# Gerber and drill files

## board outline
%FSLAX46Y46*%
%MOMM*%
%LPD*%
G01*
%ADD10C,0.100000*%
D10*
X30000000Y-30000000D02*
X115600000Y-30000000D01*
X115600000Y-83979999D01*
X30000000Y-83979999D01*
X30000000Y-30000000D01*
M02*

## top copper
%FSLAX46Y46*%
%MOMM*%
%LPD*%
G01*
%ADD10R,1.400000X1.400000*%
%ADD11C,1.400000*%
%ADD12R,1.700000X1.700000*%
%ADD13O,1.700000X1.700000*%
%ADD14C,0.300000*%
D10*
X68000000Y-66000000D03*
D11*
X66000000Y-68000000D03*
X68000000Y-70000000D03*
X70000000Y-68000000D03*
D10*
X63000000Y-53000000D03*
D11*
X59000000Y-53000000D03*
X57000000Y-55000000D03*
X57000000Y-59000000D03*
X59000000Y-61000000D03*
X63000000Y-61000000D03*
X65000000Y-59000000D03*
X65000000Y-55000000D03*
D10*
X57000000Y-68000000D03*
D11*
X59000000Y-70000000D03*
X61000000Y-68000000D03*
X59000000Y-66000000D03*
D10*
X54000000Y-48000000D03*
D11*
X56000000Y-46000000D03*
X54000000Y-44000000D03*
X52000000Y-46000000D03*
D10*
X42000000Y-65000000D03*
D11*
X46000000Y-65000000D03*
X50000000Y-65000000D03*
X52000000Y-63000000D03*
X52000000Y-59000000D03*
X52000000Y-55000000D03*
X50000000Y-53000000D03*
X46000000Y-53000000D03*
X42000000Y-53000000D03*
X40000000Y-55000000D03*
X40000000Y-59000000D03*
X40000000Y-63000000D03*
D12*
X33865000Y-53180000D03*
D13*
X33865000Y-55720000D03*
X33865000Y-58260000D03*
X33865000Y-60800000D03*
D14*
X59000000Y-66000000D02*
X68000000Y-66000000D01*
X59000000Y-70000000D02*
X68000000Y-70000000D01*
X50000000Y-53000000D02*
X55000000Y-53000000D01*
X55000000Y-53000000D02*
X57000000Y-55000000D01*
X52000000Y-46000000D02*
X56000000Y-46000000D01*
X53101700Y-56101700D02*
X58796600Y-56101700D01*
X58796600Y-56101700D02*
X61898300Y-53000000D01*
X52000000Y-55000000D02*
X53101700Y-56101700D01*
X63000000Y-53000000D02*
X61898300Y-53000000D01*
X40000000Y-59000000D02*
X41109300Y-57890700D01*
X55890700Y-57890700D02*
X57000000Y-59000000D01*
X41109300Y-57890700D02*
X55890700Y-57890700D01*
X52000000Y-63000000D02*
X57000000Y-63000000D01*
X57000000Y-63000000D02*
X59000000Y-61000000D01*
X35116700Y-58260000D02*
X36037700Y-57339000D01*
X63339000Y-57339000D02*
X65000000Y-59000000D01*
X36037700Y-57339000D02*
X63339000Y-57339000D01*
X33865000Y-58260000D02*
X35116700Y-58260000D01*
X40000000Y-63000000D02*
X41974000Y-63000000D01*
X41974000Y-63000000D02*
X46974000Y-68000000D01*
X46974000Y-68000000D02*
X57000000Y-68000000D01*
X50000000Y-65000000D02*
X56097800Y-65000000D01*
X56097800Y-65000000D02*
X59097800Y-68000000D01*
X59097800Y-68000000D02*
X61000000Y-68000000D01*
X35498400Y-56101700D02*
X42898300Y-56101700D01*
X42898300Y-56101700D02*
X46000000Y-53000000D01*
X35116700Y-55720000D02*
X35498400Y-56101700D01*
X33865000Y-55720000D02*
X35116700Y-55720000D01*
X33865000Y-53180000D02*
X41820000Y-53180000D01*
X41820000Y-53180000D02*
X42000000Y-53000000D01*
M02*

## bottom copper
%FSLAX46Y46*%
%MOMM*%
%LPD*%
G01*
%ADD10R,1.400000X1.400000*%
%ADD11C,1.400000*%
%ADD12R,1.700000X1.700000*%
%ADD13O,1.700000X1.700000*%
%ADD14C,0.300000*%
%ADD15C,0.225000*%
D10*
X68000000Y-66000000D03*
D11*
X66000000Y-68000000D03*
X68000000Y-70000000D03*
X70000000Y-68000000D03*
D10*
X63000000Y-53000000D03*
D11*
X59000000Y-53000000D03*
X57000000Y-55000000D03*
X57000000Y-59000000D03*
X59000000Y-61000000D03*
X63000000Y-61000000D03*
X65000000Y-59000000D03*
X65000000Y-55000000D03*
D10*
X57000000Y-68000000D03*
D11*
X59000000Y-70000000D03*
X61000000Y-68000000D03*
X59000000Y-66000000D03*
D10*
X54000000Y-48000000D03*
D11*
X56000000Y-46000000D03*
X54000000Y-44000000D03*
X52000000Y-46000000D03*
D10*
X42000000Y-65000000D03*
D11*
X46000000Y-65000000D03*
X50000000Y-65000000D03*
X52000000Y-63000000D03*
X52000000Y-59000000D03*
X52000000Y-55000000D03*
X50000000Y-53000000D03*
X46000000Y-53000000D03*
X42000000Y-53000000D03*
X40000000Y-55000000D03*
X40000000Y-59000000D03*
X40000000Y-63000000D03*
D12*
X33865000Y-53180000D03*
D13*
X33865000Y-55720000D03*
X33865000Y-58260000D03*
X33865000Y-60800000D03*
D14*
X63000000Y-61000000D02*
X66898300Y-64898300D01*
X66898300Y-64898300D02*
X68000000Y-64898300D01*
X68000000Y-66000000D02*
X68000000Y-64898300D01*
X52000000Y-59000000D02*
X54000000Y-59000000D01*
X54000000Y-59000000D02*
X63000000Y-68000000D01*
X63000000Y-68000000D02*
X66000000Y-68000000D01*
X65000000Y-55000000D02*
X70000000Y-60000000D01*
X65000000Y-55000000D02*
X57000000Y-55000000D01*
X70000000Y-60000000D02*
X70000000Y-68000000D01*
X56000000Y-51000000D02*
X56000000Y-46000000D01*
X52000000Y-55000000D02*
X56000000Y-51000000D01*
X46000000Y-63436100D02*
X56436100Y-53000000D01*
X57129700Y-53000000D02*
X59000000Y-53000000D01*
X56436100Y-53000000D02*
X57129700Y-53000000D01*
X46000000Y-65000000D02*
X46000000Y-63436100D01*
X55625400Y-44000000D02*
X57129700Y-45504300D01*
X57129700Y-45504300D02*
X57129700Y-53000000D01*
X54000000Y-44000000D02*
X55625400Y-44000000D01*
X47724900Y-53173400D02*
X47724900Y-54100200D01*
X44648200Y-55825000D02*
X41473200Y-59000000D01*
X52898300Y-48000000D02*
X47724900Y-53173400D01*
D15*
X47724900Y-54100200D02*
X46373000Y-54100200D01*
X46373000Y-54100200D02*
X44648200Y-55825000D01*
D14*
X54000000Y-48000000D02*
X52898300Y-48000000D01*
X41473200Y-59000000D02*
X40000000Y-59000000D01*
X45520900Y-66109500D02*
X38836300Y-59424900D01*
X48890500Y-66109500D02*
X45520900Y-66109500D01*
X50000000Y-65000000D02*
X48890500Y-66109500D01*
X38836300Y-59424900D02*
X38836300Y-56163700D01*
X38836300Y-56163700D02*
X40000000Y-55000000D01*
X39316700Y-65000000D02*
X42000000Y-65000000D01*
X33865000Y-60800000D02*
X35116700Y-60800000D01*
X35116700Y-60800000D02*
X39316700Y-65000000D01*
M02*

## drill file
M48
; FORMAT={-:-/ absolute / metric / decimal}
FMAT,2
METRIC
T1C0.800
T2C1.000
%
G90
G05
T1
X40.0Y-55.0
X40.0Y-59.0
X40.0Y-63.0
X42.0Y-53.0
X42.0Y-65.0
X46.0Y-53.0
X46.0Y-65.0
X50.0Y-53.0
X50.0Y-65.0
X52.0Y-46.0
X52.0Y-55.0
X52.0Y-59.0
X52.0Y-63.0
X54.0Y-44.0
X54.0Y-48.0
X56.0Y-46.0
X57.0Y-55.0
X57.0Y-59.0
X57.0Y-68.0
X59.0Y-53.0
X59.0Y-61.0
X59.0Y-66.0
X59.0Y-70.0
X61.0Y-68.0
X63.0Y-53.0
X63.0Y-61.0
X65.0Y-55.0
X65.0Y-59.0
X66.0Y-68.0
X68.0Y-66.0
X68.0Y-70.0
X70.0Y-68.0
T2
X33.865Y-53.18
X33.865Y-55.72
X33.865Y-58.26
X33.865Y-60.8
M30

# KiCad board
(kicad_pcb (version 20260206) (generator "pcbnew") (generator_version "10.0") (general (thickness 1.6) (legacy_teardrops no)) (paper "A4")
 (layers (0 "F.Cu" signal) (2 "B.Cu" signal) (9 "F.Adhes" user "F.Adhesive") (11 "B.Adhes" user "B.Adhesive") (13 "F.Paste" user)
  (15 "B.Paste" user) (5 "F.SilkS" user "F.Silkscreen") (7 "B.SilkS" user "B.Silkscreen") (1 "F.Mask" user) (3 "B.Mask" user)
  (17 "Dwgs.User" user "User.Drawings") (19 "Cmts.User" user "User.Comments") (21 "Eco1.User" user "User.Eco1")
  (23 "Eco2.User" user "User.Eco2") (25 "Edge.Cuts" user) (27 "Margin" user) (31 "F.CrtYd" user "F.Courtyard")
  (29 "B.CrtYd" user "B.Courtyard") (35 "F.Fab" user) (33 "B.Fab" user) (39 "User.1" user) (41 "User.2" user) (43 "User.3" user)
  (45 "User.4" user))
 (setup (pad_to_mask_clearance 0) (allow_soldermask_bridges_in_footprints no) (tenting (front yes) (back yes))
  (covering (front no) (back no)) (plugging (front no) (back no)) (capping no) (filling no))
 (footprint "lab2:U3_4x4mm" (layer "F.Cu") (at 68 68 -90)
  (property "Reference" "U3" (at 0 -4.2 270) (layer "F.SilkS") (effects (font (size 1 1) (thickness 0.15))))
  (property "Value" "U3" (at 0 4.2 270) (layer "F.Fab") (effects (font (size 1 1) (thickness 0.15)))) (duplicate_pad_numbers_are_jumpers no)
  (pad "1" thru_hole rect (at -2 0 270) (size 1.4 1.4) (drill 0.8) (layers "*.Cu" "*.Mask") (remove_unused_layers no) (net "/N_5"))
  (pad "2" thru_hole circle (at 0 2 270) (size 1.4 1.4) (drill 0.8) (layers "*.Cu" "*.Mask") (remove_unused_layers no) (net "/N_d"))
  (pad "3" thru_hole circle (at 2 0 270) (size 1.4 1.4) (drill 0.8) (layers "*.Cu" "*.Mask") (remove_unused_layers no) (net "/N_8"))
  (pad "4" thru_hole circle (at 0 -2 270) (size 1.4 1.4) (drill 0.8) (layers "*.Cu" "*.Mask") (remove_unused_layers no) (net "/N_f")))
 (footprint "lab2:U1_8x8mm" (layer "F.Cu") (at 61 57 -90)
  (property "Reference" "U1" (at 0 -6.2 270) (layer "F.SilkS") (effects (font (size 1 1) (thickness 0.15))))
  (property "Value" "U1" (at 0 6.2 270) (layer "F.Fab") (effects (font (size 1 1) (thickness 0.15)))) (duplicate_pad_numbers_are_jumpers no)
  (pad "1" thru_hole rect (at -4 -2 270) (size 1.4 1.4) (drill 0.8) (layers "*.Cu" "*.Mask") (remove_unused_layers no) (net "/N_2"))
  (pad "2" thru_hole circle (at -4 2 270) (size 1.4 1.4) (drill 0.8) (layers "*.Cu" "*.Mask") (remove_unused_layers no) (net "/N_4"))
  (pad "3" thru_hole circle (at -2 4 270) (size 1.4 1.4) (drill 0.8) (layers "*.Cu" "*.Mask") (remove_unused_layers no) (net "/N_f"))
  (pad "4" thru_hole circle (at 2 4 270) (size 1.4 1.4) (drill 0.8) (layers "*.Cu" "*.Mask") (remove_unused_layers no) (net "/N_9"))
  (pad "5" thru_hole circle (at 4 2 270) (size 1.4 1.4) (drill 0.8) (layers "*.Cu" "*.Mask") (remove_unused_layers no) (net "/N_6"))
  (pad "6" thru_hole circle (at 4 -2 270) (size 1.4 1.4) (drill 0.8) (layers "*.Cu" "*.Mask") (remove_unused_layers no) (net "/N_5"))
  (pad "7" thru_hole circle (at 2 -4 270) (size 1.4 1.4) (drill 0.8) (layers "*.Cu" "*.Mask") (remove_unused_layers no) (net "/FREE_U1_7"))
  (pad "8" thru_hole circle (at -2 -4 270) (size 1.4 1.4) (drill 0.8) (layers "*.Cu" "*.Mask") (remove_unused_layers no) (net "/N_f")))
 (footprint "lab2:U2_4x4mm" (layer "F.Cu") (at 59 68)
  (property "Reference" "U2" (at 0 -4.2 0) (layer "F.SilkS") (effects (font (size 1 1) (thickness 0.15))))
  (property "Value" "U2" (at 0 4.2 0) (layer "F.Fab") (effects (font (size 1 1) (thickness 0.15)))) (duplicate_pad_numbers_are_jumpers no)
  (pad "1" thru_hole rect (at -2 0) (size 1.4 1.4) (drill 0.8) (layers "*.Cu" "*.Mask") (remove_unused_layers no) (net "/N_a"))
  (pad "2" thru_hole circle (at 0 2) (size 1.4 1.4) (drill 0.8) (layers "*.Cu" "*.Mask") (remove_unused_layers no) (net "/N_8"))
  (pad "3" thru_hole circle (at 2 0) (size 1.4 1.4) (drill 0.8) (layers "*.Cu" "*.Mask") (remove_unused_layers no) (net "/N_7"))
  (pad "4" thru_hole circle (at 0 -2) (size 1.4 1.4) (drill 0.8) (layers "*.Cu" "*.Mask") (remove_unused_layers no) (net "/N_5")))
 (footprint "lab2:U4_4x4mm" (layer "F.Cu") (at 54 46 90)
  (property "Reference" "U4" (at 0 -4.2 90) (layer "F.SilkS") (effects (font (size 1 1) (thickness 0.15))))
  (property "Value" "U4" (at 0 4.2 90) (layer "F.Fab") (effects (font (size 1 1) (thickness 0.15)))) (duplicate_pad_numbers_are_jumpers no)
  (pad "1" thru_hole rect (at -2 0 90) (size 1.4 1.4) (drill 0.8) (layers "*.Cu" "*.Mask") (remove_unused_layers no) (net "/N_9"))
  (pad "2" thru_hole circle (at 0 2 90) (size 1.4 1.4) (drill 0.8) (layers "*.Cu" "*.Mask") (remove_unused_layers no) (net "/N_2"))
  (pad "3" thru_hole circle (at 2 0 90) (size 1.4 1.4) (drill 0.8) (layers "*.Cu" "*.Mask") (remove_unused_layers no) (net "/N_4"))
  (pad "4" thru_hole circle (at 0 -2 90) (size 1.4 1.4) (drill 0.8) (layers "*.Cu" "*.Mask") (remove_unused_layers no) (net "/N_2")))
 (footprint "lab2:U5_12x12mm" (layer "F.Cu") (at 46 59 90)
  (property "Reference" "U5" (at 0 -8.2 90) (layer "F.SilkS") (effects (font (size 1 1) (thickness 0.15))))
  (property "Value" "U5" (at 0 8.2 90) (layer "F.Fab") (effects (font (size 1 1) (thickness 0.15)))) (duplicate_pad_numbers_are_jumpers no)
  (pad "1" thru_hole rect (at -6 -4 90) (size 1.4 1.4) (drill 0.8) (layers "*.Cu" "*.Mask") (remove_unused_layers no) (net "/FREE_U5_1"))
  (pad "2" thru_hole circle (at -6 0 90) (size 1.4 1.4) (drill 0.8) (layers "*.Cu" "*.Mask") (remove_unused_layers no) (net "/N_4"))
  (pad "3" thru_hole circle (at -6 4 90) (size 1.4 1.4) (drill 0.8) (layers "*.Cu" "*.Mask") (remove_unused_layers no) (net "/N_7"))
  (pad "4" thru_hole circle (at -4 6 90) (size 1.4 1.4) (drill 0.8) (layers "*.Cu" "*.Mask") (remove_unused_layers no) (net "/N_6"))
  (pad "5" thru_hole circle (at 0 6 90) (size 1.4 1.4) (drill 0.8) (layers "*.Cu" "*.Mask") (remove_unused_layers no) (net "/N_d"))
  (pad "6" thru_hole circle (at 4 6 90) (size 1.4 1.4) (drill 0.8) (layers "*.Cu" "*.Mask") (remove_unused_layers no) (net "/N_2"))
  (pad "7" thru_hole circle (at 6 4 90) (size 1.4 1.4) (drill 0.8) (layers "*.Cu" "*.Mask") (remove_unused_layers no) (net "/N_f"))
  (pad "8" thru_hole circle (at 6 0 90) (size 1.4 1.4) (drill 0.8) (layers "*.Cu" "*.Mask") (remove_unused_layers no) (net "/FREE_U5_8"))
  (pad "9" thru_hole circle (at 6 -4 90) (size 1.4 1.4) (drill 0.8) (layers "*.Cu" "*.Mask") (remove_unused_layers no) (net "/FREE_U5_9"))
  (pad "10" thru_hole circle (at 4 -6 90) (size 1.4 1.4) (drill 0.8) (layers "*.Cu" "*.Mask") (remove_unused_layers no) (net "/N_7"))
  (pad "11" thru_hole circle (at 0 -6 90) (size 1.4 1.4) (drill 0.8) (layers "*.Cu" "*.Mask") (remove_unused_layers no) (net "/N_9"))
  (pad "12" thru_hole circle (at -4 -6 90) (size 1.4 1.4) (drill 0.8) (layers "*.Cu" "*.Mask") (remove_unused_layers no) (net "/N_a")))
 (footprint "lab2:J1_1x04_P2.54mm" (layer "F.Cu") (at 33.865 56.99)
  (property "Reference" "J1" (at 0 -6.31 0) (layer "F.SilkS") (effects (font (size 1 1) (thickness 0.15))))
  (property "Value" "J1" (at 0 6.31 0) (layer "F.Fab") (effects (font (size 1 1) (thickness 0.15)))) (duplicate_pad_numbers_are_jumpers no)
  (pad "1" thru_hole rect (at 0 -3.81) (size 1.7 1.7) (drill 1) (layers "*.Cu" "*.Mask") (remove_unused_layers no) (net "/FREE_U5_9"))
  (pad "2" thru_hole oval (at 0 -1.27) (size 1.7 1.7) (drill 1) (layers "*.Cu" "*.Mask") (remove_unused_layers no) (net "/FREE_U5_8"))
  (pad "3" thru_hole oval (at 0 1.27) (size 1.7 1.7) (drill 1) (layers "*.Cu" "*.Mask") (remove_unused_layers no) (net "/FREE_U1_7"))
  (pad "4" thru_hole oval (at 0 3.81) (size 1.7 1.7) (drill 1) (layers "*.Cu" "*.Mask") (remove_unused_layers no) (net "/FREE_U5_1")))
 (gr_rect (start 30 30) (end 115.6 83.979999) (stroke (width 0.1) (type default)) (fill no) (layer "Edge.Cuts"))
 (segment (start 59 66) (end 68 66) (width 0.3) (layer "F.Cu") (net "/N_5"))
 (segment (start 63 61) (end 66.8983 64.8983) (width 0.3) (layer "B.Cu") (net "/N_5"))
 (segment (start 66.8983 64.8983) (end 68 64.8983) (width 0.3) (layer "B.Cu") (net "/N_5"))
 (segment (start 68 66) (end 68 64.8983) (width 0.3) (layer "B.Cu") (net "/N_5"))
 (segment (start 52 59) (end 54 59) (width 0.3) (layer "B.Cu") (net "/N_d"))
 (segment (start 54 59) (end 63 68) (width 0.3) (layer "B.Cu") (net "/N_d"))
 (segment (start 63 68) (end 66 68) (width 0.3) (layer "B.Cu") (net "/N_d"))
 (segment (start 59 70) (end 68 70) (width 0.3) (layer "F.Cu") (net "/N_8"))
 (segment (start 50 53) (end 55 53) (width 0.3) (layer "F.Cu") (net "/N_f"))
 (segment (start 55 53) (end 57 55) (width 0.3) (layer "F.Cu") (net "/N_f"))
 (segment (start 65 55) (end 70 60) (width 0.3) (layer "B.Cu") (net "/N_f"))
 (segment (start 65 55) (end 57 55) (width 0.3) (layer "B.Cu") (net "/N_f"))
 (segment (start 70 60) (end 70 68) (width 0.3) (layer "B.Cu") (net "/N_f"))
 (segment (start 52 46) (end 56 46) (width 0.3) (layer "F.Cu") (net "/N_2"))
 (segment (start 53.1017 56.1017) (end 58.7966 56.1017) (width 0.3) (layer "F.Cu") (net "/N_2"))
 (segment (start 58.7966 56.1017) (end 61.8983 53) (width 0.3) (layer "F.Cu") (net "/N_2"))
 (segment (start 52 55) (end 53.1017 56.1017) (width 0.3) (layer "F.Cu") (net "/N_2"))
 (segment (start 63 53) (end 61.8983 53) (width 0.3) (layer "F.Cu") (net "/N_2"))
 (segment (start 56 51) (end 56 46) (width 0.3) (layer "B.Cu") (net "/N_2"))
 (segment (start 52 55) (end 56 51) (width 0.3) (layer "B.Cu") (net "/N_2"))
 (segment (start 46 63.4361) (end 56.4361 53) (width 0.3) (layer "B.Cu") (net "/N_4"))
 (segment (start 57.1297 53) (end 59 53) (width 0.3) (layer "B.Cu") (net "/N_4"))
 (segment (start 56.4361 53) (end 57.1297 53) (width 0.3) (layer "B.Cu") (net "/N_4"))
 (segment (start 46 65) (end 46 63.4361) (width 0.3) (layer "B.Cu") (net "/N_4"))
 (segment (start 55.6254 44) (end 57.1297 45.5043) (width 0.3) (layer "B.Cu") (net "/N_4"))
 (segment (start 57.1297 45.5043) (end 57.1297 53) (width 0.3) (layer "B.Cu") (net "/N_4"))
 (segment (start 54 44) (end 55.6254 44) (width 0.3) (layer "B.Cu") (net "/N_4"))
 (segment (start 40 59) (end 41.1093 57.8907) (width 0.3) (layer "F.Cu") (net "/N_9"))
 (segment (start 55.8907 57.8907) (end 57 59) (width 0.3) (layer "F.Cu") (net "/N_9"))
 (segment (start 41.1093 57.8907) (end 55.8907 57.8907) (width 0.3) (layer "F.Cu") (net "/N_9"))
 (segment (start 47.7249 53.1734) (end 47.7249 54.1002) (width 0.3) (layer "B.Cu") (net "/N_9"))
 (segment (start 44.6482 55.825) (end 41.4732 59) (width 0.3) (layer "B.Cu") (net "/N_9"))
 (segment (start 52.8983 48) (end 47.7249 53.1734) (width 0.3) (layer "B.Cu") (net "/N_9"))
 (segment (start 47.7249 54.1002) (end 46.373 54.1002) (width 0.225) (layer "B.Cu") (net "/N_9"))
 (segment (start 46.373 54.1002) (end 44.6482 55.825) (width 0.225) (layer "B.Cu") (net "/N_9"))
 (segment (start 54 48) (end 52.8983 48) (width 0.3) (layer "B.Cu") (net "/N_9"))
 (segment (start 41.4732 59) (end 40 59) (width 0.3) (layer "B.Cu") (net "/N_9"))
 (segment (start 52 63) (end 57 63) (width 0.3) (layer "F.Cu") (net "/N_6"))
 (segment (start 57 63) (end 59 61) (width 0.3) (layer "F.Cu") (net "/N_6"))
 (segment (start 35.1167 58.26) (end 36.0377 57.339) (width 0.3) (layer "F.Cu") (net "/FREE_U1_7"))
 (segment (start 63.339 57.339) (end 65 59) (width 0.3) (layer "F.Cu") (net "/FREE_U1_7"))
 (segment (start 36.0377 57.339) (end 63.339 57.339) (width 0.3) (layer "F.Cu") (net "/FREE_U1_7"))
 (segment (start 33.865 58.26) (end 35.1167 58.26) (width 0.3) (layer "F.Cu") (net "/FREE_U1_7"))
 (segment (start 40 63) (end 41.974 63) (width 0.3) (layer "F.Cu") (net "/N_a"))
 (segment (start 41.974 63) (end 46.974 68) (width 0.3) (layer "F.Cu") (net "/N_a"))
 (segment (start 46.974 68) (end 57 68) (width 0.3) (layer "F.Cu") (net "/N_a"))
 (segment (start 50 65) (end 56.0978 65) (width 0.3) (layer "F.Cu") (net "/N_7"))
 (segment (start 56.0978 65) (end 59.0978 68) (width 0.3) (layer "F.Cu") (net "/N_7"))
 (segment (start 59.0978 68) (end 61 68) (width 0.3) (layer "F.Cu") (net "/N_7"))
 (segment (start 45.5209 66.1095) (end 38.8363 59.4249) (width 0.3) (layer "B.Cu") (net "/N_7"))
 (segment (start 48.8905 66.1095) (end 45.5209 66.1095) (width 0.3) (layer "B.Cu") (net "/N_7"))
 (segment (start 50 65) (end 48.8905 66.1095) (width 0.3) (layer "B.Cu") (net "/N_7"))
 (segment (start 38.8363 59.4249) (end 38.8363 56.1637) (width 0.3) (layer "B.Cu") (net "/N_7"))
 (segment (start 38.8363 56.1637) (end 40 55) (width 0.3) (layer "B.Cu") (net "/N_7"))
 (segment (start 39.3167 65) (end 42 65) (width 0.3) (layer "B.Cu") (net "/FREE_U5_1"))
 (segment (start 33.865 60.8) (end 35.1167 60.8) (width 0.3) (layer "B.Cu") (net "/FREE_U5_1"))
 (segment (start 35.1167 60.8) (end 39.3167 65) (width 0.3) (layer "B.Cu") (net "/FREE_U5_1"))
 (segment (start 35.4984 56.1017) (end 42.8983 56.1017) (width 0.3) (layer "F.Cu") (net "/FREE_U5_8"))
 (segment (start 42.8983 56.1017) (end 46 53) (width 0.3) (layer "F.Cu") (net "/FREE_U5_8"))
 (segment (start 35.1167 55.72) (end 35.4984 56.1017) (width 0.3) (layer "F.Cu") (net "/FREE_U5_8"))
 (segment (start 33.865 55.72) (end 35.1167 55.72) (width 0.3) (layer "F.Cu") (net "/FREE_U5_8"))
 (segment (start 33.865 53.18) (end 41.82 53.18) (width 0.3) (layer "F.Cu") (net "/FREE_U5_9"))
 (segment (start 41.82 53.18) (end 42 53) (width 0.3) (layer "F.Cu") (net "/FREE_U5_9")))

